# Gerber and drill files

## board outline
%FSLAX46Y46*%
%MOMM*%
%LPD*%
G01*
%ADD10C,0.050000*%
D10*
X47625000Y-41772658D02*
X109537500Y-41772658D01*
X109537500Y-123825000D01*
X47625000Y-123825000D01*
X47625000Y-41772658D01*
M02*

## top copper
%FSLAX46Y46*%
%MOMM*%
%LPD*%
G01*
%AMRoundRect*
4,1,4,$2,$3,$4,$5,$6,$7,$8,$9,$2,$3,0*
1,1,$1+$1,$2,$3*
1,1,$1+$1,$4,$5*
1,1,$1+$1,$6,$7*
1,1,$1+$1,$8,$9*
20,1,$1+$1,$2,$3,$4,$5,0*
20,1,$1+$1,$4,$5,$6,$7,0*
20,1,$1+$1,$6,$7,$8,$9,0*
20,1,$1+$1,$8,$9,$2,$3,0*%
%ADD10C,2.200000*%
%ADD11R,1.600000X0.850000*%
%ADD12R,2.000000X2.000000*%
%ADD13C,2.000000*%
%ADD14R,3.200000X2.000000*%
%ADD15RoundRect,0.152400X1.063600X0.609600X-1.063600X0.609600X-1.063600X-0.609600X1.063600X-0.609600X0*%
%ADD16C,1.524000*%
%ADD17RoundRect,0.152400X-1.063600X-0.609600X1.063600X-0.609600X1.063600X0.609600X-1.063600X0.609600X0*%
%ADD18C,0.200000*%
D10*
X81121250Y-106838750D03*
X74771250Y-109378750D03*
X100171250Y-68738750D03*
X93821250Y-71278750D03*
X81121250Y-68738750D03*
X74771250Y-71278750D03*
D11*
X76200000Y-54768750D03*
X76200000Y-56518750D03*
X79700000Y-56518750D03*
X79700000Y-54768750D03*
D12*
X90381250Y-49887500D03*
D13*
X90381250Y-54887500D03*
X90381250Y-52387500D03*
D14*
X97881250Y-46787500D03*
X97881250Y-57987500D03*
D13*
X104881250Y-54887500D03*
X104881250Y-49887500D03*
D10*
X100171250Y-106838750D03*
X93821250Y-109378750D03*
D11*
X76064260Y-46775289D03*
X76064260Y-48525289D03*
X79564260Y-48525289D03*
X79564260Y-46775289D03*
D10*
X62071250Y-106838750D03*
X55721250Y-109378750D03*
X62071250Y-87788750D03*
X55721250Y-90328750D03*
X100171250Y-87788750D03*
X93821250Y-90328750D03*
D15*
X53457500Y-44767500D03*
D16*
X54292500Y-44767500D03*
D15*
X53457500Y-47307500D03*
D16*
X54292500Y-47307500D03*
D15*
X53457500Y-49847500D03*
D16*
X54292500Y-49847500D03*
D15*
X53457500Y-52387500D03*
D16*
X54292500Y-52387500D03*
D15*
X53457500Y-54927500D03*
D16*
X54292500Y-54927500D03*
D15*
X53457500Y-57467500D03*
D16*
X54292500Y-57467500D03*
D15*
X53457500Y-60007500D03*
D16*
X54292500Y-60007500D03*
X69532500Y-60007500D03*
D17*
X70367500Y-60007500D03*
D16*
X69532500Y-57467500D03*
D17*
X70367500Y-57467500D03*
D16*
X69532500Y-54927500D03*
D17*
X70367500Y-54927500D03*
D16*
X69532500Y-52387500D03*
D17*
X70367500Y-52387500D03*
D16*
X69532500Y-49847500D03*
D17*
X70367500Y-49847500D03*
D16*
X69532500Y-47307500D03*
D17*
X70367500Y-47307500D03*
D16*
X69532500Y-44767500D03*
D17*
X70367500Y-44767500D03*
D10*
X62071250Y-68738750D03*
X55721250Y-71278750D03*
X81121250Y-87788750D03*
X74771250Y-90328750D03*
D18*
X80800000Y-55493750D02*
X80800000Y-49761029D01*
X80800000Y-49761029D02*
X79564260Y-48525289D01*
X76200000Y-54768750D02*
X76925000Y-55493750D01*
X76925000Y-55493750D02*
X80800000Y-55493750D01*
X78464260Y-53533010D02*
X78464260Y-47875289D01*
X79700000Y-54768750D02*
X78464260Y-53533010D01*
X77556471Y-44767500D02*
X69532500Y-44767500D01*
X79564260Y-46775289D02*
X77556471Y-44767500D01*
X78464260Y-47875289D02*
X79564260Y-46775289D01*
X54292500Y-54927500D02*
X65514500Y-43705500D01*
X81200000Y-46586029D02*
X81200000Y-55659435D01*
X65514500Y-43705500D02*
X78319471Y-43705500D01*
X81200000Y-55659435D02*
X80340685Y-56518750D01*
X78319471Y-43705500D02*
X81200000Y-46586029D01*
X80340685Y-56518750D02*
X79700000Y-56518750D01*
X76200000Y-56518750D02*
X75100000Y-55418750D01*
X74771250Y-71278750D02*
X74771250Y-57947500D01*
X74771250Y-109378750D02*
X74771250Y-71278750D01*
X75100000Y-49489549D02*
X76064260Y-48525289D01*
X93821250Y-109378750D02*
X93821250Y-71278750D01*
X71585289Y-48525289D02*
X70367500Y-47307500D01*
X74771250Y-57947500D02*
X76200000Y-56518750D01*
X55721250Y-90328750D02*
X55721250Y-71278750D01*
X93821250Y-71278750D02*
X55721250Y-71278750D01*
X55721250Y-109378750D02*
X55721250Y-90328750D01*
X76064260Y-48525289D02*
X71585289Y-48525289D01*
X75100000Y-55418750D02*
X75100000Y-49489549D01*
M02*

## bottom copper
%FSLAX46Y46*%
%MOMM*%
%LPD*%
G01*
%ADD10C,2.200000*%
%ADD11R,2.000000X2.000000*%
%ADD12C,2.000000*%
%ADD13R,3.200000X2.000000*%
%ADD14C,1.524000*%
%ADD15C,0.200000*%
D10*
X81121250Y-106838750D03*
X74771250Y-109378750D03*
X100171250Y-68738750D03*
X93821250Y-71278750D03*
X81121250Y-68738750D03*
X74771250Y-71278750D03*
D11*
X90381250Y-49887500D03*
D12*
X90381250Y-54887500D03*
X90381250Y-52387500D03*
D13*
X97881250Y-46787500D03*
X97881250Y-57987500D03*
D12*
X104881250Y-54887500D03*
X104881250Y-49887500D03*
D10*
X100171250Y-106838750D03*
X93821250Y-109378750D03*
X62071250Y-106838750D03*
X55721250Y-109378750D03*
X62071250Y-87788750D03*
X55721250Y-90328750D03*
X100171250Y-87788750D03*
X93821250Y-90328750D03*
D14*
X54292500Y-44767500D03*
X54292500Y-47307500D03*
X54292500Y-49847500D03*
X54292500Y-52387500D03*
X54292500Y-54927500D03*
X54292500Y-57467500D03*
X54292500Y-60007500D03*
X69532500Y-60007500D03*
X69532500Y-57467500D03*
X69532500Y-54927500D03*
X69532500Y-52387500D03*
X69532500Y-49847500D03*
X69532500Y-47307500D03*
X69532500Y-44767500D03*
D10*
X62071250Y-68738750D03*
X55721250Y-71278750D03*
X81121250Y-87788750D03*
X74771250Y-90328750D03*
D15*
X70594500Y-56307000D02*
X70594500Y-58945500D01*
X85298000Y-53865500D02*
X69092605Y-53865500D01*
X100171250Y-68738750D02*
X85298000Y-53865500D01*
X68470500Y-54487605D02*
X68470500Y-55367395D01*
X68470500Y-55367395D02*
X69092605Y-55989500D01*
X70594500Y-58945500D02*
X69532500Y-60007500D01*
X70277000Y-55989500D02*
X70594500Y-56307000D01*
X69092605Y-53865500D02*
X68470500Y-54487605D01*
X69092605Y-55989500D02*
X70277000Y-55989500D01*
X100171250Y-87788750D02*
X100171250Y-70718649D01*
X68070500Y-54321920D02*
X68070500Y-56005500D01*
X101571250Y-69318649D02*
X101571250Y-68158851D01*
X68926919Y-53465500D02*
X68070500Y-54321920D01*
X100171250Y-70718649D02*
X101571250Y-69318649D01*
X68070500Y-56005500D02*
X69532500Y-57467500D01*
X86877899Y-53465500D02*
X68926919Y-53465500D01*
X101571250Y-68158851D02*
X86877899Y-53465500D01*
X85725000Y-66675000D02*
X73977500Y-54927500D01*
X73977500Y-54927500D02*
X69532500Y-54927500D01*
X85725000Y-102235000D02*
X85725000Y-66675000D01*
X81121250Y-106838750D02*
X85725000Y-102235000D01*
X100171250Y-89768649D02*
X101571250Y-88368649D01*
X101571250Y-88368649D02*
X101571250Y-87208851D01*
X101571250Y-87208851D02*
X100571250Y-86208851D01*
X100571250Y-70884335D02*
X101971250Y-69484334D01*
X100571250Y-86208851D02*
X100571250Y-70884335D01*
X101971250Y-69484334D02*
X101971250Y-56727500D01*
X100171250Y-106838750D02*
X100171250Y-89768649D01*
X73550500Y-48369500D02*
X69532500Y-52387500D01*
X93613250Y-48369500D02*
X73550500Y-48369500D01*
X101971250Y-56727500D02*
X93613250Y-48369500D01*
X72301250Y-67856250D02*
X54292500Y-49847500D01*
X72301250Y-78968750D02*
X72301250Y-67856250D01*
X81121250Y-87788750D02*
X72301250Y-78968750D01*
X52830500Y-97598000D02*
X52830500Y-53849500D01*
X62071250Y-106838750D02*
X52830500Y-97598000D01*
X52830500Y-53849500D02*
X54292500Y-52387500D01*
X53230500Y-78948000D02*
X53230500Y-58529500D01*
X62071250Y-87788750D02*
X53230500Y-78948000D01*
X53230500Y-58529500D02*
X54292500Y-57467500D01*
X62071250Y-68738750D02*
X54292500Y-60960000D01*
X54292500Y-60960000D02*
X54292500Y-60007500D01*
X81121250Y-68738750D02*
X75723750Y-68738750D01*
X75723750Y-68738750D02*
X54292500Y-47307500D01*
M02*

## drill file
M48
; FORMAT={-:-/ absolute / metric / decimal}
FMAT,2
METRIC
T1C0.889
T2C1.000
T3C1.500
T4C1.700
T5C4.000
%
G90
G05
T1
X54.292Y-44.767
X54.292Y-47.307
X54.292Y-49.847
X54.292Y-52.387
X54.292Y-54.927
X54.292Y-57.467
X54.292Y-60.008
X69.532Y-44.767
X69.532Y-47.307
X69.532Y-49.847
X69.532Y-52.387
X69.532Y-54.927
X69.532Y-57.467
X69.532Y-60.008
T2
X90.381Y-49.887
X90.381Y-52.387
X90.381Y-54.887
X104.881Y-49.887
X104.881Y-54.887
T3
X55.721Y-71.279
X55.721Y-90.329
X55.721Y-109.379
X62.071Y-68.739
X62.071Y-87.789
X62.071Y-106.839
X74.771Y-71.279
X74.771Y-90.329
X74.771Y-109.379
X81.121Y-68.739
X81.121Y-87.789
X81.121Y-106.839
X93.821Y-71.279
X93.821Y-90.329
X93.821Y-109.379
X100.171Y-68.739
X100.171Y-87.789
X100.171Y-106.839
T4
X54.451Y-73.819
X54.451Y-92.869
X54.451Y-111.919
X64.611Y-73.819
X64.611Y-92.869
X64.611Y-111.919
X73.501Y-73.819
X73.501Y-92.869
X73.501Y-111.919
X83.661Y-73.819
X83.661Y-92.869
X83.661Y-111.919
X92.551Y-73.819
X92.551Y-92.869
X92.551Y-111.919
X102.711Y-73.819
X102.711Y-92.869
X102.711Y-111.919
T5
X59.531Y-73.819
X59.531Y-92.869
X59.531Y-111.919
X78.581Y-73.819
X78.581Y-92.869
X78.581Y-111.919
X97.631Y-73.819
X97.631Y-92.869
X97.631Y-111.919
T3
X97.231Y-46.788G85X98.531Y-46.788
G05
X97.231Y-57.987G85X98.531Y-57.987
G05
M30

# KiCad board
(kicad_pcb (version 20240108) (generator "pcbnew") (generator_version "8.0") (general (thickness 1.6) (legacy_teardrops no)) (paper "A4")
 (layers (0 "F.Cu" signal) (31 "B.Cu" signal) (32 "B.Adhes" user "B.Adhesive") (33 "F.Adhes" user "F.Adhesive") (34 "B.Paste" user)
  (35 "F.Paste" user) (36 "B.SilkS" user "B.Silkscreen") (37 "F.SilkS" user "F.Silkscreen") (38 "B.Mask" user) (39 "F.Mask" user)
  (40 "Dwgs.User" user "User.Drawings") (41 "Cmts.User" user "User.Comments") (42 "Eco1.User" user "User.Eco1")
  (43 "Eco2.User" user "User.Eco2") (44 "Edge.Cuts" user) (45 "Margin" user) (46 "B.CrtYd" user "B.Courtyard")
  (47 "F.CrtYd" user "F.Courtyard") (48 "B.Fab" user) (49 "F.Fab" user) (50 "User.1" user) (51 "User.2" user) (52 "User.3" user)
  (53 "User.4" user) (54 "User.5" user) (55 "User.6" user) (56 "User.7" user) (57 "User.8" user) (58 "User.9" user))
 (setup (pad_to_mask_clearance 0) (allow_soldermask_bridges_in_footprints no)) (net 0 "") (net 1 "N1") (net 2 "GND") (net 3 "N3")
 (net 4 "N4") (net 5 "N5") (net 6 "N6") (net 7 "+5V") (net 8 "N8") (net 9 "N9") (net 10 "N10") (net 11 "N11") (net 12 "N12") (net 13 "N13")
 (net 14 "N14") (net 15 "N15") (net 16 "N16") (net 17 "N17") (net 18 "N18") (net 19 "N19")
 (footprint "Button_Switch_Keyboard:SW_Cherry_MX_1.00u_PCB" (layer "F.Cu") (at 81.12125 106.83875)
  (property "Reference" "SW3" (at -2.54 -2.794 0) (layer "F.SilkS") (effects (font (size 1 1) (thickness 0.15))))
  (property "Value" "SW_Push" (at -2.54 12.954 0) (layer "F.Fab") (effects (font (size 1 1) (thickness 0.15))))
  (pad "" np_thru_hole circle (at -7.62 5.08) (size 1.7 1.7) (drill 1.7) (layers "*.Cu" "*.Mask"))
  (pad "" np_thru_hole circle (at -2.54 5.08) (size 4 4) (drill 4) (layers "*.Cu" "*.Mask"))
  (pad "" np_thru_hole circle (at 2.54 5.08) (size 1.7 1.7) (drill 1.7) (layers "*.Cu" "*.Mask"))
  (pad "1" thru_hole circle (at 0 0) (size 2.2 2.2) (drill 1.5) (layers "*.Cu" "*.Mask") (remove_unused_layers no) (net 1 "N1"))
  (pad "2" thru_hole circle (at -6.35 2.54) (size 2.2 2.2) (drill 1.5) (layers "*.Cu" "*.Mask") (remove_unused_layers no) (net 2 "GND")))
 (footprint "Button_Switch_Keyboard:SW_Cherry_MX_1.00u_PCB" (layer "F.Cu") (at 100.17125 68.73875)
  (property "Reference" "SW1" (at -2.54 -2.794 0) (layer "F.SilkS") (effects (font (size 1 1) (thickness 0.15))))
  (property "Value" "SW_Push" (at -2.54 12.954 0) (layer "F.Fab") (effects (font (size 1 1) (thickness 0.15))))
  (pad "" np_thru_hole circle (at -7.62 5.08) (size 1.7 1.7) (drill 1.7) (layers "*.Cu" "*.Mask"))
  (pad "" np_thru_hole circle (at -2.54 5.08) (size 4 4) (drill 4) (layers "*.Cu" "*.Mask"))
  (pad "" np_thru_hole circle (at 2.54 5.08) (size 1.7 1.7) (drill 1.7) (layers "*.Cu" "*.Mask"))
  (pad "1" thru_hole circle (at 0 0) (size 2.2 2.2) (drill 1.5) (layers "*.Cu" "*.Mask") (remove_unused_layers no) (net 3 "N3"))
  (pad "2" thru_hole circle (at -6.35 2.54) (size 2.2 2.2) (drill 1.5) (layers "*.Cu" "*.Mask") (remove_unused_layers no) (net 2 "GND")))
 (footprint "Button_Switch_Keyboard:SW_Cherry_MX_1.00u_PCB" (layer "F.Cu") (at 81.12125 68.73875)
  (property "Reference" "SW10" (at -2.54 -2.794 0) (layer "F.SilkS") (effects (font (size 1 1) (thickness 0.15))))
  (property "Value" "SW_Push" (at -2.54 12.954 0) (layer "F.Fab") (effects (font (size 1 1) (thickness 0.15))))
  (pad "" np_thru_hole circle (at -7.62 5.08) (size 1.7 1.7) (drill 1.7) (layers "*.Cu" "*.Mask"))
  (pad "" np_thru_hole circle (at -2.54 5.08) (size 4 4) (drill 4) (layers "*.Cu" "*.Mask"))
  (pad "" np_thru_hole circle (at 2.54 5.08) (size 1.7 1.7) (drill 1.7) (layers "*.Cu" "*.Mask"))
  (pad "1" thru_hole circle (at 0 0) (size 2.2 2.2) (drill 1.5) (layers "*.Cu" "*.Mask") (remove_unused_layers no) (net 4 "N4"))
  (pad "2" thru_hole circle (at -6.35 2.54) (size 2.2 2.2) (drill 1.5) (layers "*.Cu" "*.Mask") (remove_unused_layers no) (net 2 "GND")))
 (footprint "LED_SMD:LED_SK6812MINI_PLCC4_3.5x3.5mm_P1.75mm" (layer "F.Cu") (at 77.95 55.64375)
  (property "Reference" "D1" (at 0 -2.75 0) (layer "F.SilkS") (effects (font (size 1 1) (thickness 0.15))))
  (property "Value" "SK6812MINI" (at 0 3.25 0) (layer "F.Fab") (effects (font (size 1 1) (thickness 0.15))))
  (pad "1" smd rect (at -1.75 -0.875) (size 1.6 0.85) (layers "F.Cu" "F.Paste" "F.Mask") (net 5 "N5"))
  (pad "2" smd rect (at -1.75 0.875) (size 1.6 0.85) (layers "F.Cu" "F.Paste" "F.Mask") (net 2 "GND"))
  (pad "3" smd rect (at 1.75 0.875) (size 1.6 0.85) (layers "F.Cu" "F.Paste" "F.Mask") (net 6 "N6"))
  (pad "4" smd rect (at 1.75 -0.875) (size 1.6 0.85) (layers "F.Cu" "F.Paste" "F.Mask") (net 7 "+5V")))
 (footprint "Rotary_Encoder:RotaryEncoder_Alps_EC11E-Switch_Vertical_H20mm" (layer "F.Cu") (at 90.38125 49.8875)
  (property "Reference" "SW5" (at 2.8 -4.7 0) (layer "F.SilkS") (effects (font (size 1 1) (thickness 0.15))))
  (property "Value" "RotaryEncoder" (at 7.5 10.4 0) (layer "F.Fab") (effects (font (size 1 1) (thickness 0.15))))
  (pad "A" thru_hole rect (at 0 0) (size 2 2) (drill 1) (layers "*.Cu" "*.Mask") (remove_unused_layers no) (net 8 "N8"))
  (pad "B" thru_hole circle (at 0 5) (size 2 2) (drill 1) (layers "*.Cu" "*.Mask") (remove_unused_layers no) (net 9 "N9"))
  (pad "C" thru_hole circle (at 0 2.5) (size 2 2) (drill 1) (layers "*.Cu" "*.Mask") (remove_unused_layers no) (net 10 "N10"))
  (pad "MP" thru_hole rect (at 7.5 -3.1) (size 3.2 2) (drill oval 2.8 1.5) (layers "*.Cu" "*.Mask") (remove_unused_layers no))
  (pad "MP" thru_hole rect (at 7.5 8.1) (size 3.2 2) (drill oval 2.8 1.5) (layers "*.Cu" "*.Mask") (remove_unused_layers no))
  (pad "S1" thru_hole circle (at 14.5 5) (size 2 2) (drill 1) (layers "*.Cu" "*.Mask") (remove_unused_layers no))
  (pad "S2" thru_hole circle (at 14.5 0) (size 2 2) (drill 1) (layers "*.Cu" "*.Mask") (remove_unused_layers no)))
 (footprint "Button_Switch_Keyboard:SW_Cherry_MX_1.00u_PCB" (layer "F.Cu") (at 100.17125 106.83875)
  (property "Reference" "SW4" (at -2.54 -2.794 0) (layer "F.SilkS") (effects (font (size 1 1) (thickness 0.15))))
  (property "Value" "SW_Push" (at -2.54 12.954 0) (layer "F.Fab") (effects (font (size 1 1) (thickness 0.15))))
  (pad "" np_thru_hole circle (at -7.62 5.08) (size 1.7 1.7) (drill 1.7) (layers "*.Cu" "*.Mask"))
  (pad "" np_thru_hole circle (at -2.54 5.08) (size 4 4) (drill 4) (layers "*.Cu" "*.Mask"))
  (pad "" np_thru_hole circle (at 2.54 5.08) (size 1.7 1.7) (drill 1.7) (layers "*.Cu" "*.Mask"))
  (pad "1" thru_hole circle (at 0 0) (size 2.2 2.2) (drill 1.5) (layers "*.Cu" "*.Mask") (remove_unused_layers no) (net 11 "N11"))
  (pad "2" thru_hole circle (at -6.35 2.54) (size 2.2 2.2) (drill 1.5) (layers "*.Cu" "*.Mask") (remove_unused_layers no) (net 2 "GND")))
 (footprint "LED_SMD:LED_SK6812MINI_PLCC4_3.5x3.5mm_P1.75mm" (layer "F.Cu") (at 77.81426 47.650289)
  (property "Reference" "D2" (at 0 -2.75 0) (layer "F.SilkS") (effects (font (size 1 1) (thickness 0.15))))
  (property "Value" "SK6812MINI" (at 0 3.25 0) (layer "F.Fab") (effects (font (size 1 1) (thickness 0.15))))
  (pad "1" smd rect (at -1.75 -0.875) (size 1.6 0.85) (layers "F.Cu" "F.Paste" "F.Mask") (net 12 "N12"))
  (pad "2" smd rect (at -1.75 0.875) (size 1.6 0.85) (layers "F.Cu" "F.Paste" "F.Mask") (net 2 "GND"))
  (pad "3" smd rect (at 1.75 0.875) (size 1.6 0.85) (layers "F.Cu" "F.Paste" "F.Mask") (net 5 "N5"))
  (pad "4" smd rect (at 1.75 -0.875) (size 1.6 0.85) (layers "F.Cu" "F.Paste" "F.Mask") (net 7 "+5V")))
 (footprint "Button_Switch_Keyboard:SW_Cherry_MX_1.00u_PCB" (layer "F.Cu") (at 62.07125 106.83875)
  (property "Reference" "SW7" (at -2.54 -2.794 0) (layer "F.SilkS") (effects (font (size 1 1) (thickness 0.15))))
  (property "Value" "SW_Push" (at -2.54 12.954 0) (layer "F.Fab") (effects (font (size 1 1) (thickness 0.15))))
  (pad "" np_thru_hole circle (at -7.62 5.08) (size 1.7 1.7) (drill 1.7) (layers "*.Cu" "*.Mask"))
  (pad "" np_thru_hole circle (at -2.54 5.08) (size 4 4) (drill 4) (layers "*.Cu" "*.Mask"))
  (pad "" np_thru_hole circle (at 2.54 5.08) (size 1.7 1.7) (drill 1.7) (layers "*.Cu" "*.Mask"))
  (pad "1" thru_hole circle (at 0 0) (size 2.2 2.2) (drill 1.5) (layers "*.Cu" "*.Mask") (remove_unused_layers no) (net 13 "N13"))
  (pad "2" thru_hole circle (at -6.35 2.54) (size 2.2 2.2) (drill 1.5) (layers "*.Cu" "*.Mask") (remove_unused_layers no) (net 2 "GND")))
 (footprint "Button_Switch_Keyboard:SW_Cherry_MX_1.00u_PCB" (layer "F.Cu") (at 62.07125 87.78875)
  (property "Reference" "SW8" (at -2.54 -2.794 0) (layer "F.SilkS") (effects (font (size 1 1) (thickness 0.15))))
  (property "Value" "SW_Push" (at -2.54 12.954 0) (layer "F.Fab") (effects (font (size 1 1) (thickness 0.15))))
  (pad "" np_thru_hole circle (at -7.62 5.08) (size 1.7 1.7) (drill 1.7) (layers "*.Cu" "*.Mask"))
  (pad "" np_thru_hole circle (at -2.54 5.08) (size 4 4) (drill 4) (layers "*.Cu" "*.Mask"))
  (pad "" np_thru_hole circle (at 2.54 5.08) (size 1.7 1.7) (drill 1.7) (layers "*.Cu" "*.Mask"))
  (pad "1" thru_hole circle (at 0 0) (size 2.2 2.2) (drill 1.5) (layers "*.Cu" "*.Mask") (remove_unused_layers no) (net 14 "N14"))
  (pad "2" thru_hole circle (at -6.35 2.54) (size 2.2 2.2) (drill 1.5) (layers "*.Cu" "*.Mask") (remove_unused_layers no) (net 2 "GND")))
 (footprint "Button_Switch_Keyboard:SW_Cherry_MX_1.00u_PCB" (layer "F.Cu") (at 100.17125 87.78875)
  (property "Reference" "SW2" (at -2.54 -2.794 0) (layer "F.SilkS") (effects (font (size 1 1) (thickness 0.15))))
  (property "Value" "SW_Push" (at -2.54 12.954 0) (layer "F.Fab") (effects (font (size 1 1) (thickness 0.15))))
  (pad "" np_thru_hole circle (at -7.62 5.08) (size 1.7 1.7) (drill 1.7) (layers "*.Cu" "*.Mask"))
  (pad "" np_thru_hole circle (at -2.54 5.08) (size 4 4) (drill 4) (layers "*.Cu" "*.Mask"))
  (pad "" np_thru_hole circle (at 2.54 5.08) (size 1.7 1.7) (drill 1.7) (layers "*.Cu" "*.Mask"))
  (pad "1" thru_hole circle (at 0 0) (size 2.2 2.2) (drill 1.5) (layers "*.Cu" "*.Mask") (remove_unused_layers no) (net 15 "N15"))
  (pad "2" thru_hole circle (at -6.35 2.54) (size 2.2 2.2) (drill 1.5) (layers "*.Cu" "*.Mask") (remove_unused_layers no) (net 2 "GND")))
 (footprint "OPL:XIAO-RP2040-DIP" (layer "F.Cu") (at 61.9125 52.3875)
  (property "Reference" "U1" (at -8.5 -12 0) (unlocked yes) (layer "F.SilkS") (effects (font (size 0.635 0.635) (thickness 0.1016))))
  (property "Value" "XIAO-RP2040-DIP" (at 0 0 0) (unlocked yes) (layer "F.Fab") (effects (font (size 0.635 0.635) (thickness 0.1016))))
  (pad "1" smd roundrect (at -8.455 -7.62 180) (size 2.432 1.524) (layers "F.Cu" "F.Mask") (roundrect_rratio 0.1) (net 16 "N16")
   (thermal_bridge_angle 45))
  (pad "1" thru_hole circle (at -7.62 -7.62 180) (size 1.524 1.524) (drill 0.889) (layers "*.Cu" "*.Mask") (remove_unused_layers no)
   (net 16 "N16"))
  (pad "2" smd roundrect (at -8.455 -5.08 180) (size 2.432 1.524) (layers "F.Cu" "F.Mask") (roundrect_rratio 0.1) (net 4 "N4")
   (thermal_bridge_angle 45))
  (pad "2" thru_hole circle (at -7.62 -5.08 180) (size 1.524 1.524) (drill 0.889) (layers "*.Cu" "*.Mask") (remove_unused_layers no)
   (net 4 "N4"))
  (pad "3" smd roundrect (at -8.455 -2.54 180) (size 2.432 1.524) (layers "F.Cu" "F.Mask") (roundrect_rratio 0.1) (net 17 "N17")
   (thermal_bridge_angle 45))
  (pad "3" thru_hole circle (at -7.62 -2.54 180) (size 1.524 1.524) (drill 0.889) (layers "*.Cu" "*.Mask") (remove_unused_layers no)
   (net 17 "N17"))
  (pad "4" smd roundrect (at -8.455 0 180) (size 2.432 1.524) (layers "F.Cu" "F.Mask") (roundrect_rratio 0.1) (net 13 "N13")
   (thermal_bridge_angle 45))
  (pad "4" thru_hole circle (at -7.62 0 180) (size 1.524 1.524) (drill 0.889) (layers "*.Cu" "*.Mask") (remove_unused_layers no)
   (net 13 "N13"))
  (pad "5" smd roundrect (at -8.455 2.54 180) (size 2.432 1.524) (layers "F.Cu" "F.Mask") (roundrect_rratio 0.1) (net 6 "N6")
   (thermal_bridge_angle 45))
  (pad "5" thru_hole circle (at -7.62 2.54 180) (size 1.524 1.524) (drill 0.889) (layers "*.Cu" "*.Mask") (remove_unused_layers no)
   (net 6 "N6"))
  (pad "6" smd roundrect (at -8.455 5.08 180) (size 2.432 1.524) (layers "F.Cu" "F.Mask") (roundrect_rratio 0.1) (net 14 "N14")
   (thermal_bridge_angle 45))
  (pad "6" thru_hole circle (at -7.62 5.08 180) (size 1.524 1.524) (drill 0.889) (layers "*.Cu" "*.Mask") (remove_unused_layers no)
   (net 14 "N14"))
  (pad "7" smd roundrect (at -8.455 7.62 180) (size 2.432 1.524) (layers "F.Cu" "F.Mask") (roundrect_rratio 0.1) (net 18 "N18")
   (thermal_bridge_angle 45))
  (pad "7" thru_hole circle (at -7.62 7.62 180) (size 1.524 1.524) (drill 0.889) (layers "*.Cu" "*.Mask") (remove_unused_layers no)
   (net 18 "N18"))
  (pad "8" thru_hole circle (at 7.62 7.62) (size 1.524 1.524) (drill 0.889) (layers "*.Cu" "*.Mask") (remove_unused_layers no) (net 3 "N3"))
  (pad "8" smd roundrect (at 8.455 7.62) (size 2.432 1.524) (layers "F.Cu" "F.Mask") (roundrect_rratio 0.1) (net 3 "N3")
   (thermal_bridge_angle 45))
  (pad "9" thru_hole circle (at 7.62 5.08) (size 1.524 1.524) (drill 0.889) (layers "*.Cu" "*.Mask") (remove_unused_layers no)
   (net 15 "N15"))
  (pad "9" smd roundrect (at 8.455 5.08) (size 2.432 1.524) (layers "F.Cu" "F.Mask") (roundrect_rratio 0.1) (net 15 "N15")
   (thermal_bridge_angle 45))
  (pad "10" thru_hole circle (at 7.62 2.54) (size 1.524 1.524) (drill 0.889) (layers "*.Cu" "*.Mask") (remove_unused_layers no) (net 1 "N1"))
  (pad "10" smd roundrect (at 8.455 2.54) (size 2.432 1.524) (layers "F.Cu" "F.Mask") (roundrect_rratio 0.1) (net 1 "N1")
   (thermal_bridge_angle 45))
  (pad "11" thru_hole circle (at 7.62 0) (size 1.524 1.524) (drill 0.889) (layers "*.Cu" "*.Mask") (remove_unused_layers no) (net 11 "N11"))
  (pad "11" smd roundrect (at 8.455 0) (size 2.432 1.524) (layers "F.Cu" "F.Mask") (roundrect_rratio 0.1) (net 11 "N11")
   (thermal_bridge_angle 45))
  (pad "12" thru_hole circle (at 7.62 -2.54) (size 1.524 1.524) (drill 0.889) (layers "*.Cu" "*.Mask") (remove_unused_layers no)
   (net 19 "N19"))
  (pad "12" smd roundrect (at 8.455 -2.54) (size 2.432 1.524) (layers "F.Cu" "F.Mask") (roundrect_rratio 0.1) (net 19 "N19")
   (thermal_bridge_angle 45))
  (pad "13" thru_hole circle (at 7.62 -5.08) (size 1.524 1.524) (drill 0.889) (layers "*.Cu" "*.Mask") (remove_unused_layers no)
   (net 2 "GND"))
  (pad "13" smd roundrect (at 8.455 -5.08) (size 2.432 1.524) (layers "F.Cu" "F.Mask") (roundrect_rratio 0.1) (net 2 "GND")
   (thermal_bridge_angle 45))
  (pad "14" thru_hole circle (at 7.62 -7.62) (size 1.524 1.524) (drill 0.889) (layers "*.Cu" "*.Mask") (remove_unused_layers no)
   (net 7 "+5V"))
  (pad "14" smd roundrect (at 8.455 -7.62) (size 2.432 1.524) (layers "F.Cu" "F.Mask") (roundrect_rratio 0.1) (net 7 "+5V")
   (thermal_bridge_angle 45)))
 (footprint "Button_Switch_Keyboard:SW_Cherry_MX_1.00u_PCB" (layer "F.Cu") (at 62.07125 68.73875)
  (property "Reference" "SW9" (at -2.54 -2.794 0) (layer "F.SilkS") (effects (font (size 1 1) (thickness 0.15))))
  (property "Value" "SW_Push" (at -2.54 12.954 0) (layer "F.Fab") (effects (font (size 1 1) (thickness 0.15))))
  (pad "" np_thru_hole circle (at -7.62 5.08) (size 1.7 1.7) (drill 1.7) (layers "*.Cu" "*.Mask"))
  (pad "" np_thru_hole circle (at -2.54 5.08) (size 4 4) (drill 4) (layers "*.Cu" "*.Mask"))
  (pad "" np_thru_hole circle (at 2.54 5.08) (size 1.7 1.7) (drill 1.7) (layers "*.Cu" "*.Mask"))
  (pad "1" thru_hole circle (at 0 0) (size 2.2 2.2) (drill 1.5) (layers "*.Cu" "*.Mask") (remove_unused_layers no) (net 18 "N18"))
  (pad "2" thru_hole circle (at -6.35 2.54) (size 2.2 2.2) (drill 1.5) (layers "*.Cu" "*.Mask") (remove_unused_layers no) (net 2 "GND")))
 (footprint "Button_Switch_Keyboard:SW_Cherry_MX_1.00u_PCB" (layer "F.Cu") (at 81.12125 87.78875)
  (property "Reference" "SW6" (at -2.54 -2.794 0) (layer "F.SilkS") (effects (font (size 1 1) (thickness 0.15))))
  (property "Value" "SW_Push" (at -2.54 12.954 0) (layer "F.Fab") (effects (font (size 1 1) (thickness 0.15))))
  (pad "" np_thru_hole circle (at -7.62 5.08) (size 1.7 1.7) (drill 1.7) (layers "*.Cu" "*.Mask"))
  (pad "" np_thru_hole circle (at -2.54 5.08) (size 4 4) (drill 4) (layers "*.Cu" "*.Mask"))
  (pad "" np_thru_hole circle (at 2.54 5.08) (size 1.7 1.7) (drill 1.7) (layers "*.Cu" "*.Mask"))
  (pad "1" thru_hole circle (at 0 0) (size 2.2 2.2) (drill 1.5) (layers "*.Cu" "*.Mask") (remove_unused_layers no) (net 17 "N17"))
  (pad "2" thru_hole circle (at -6.35 2.54) (size 2.2 2.2) (drill 1.5) (layers "*.Cu" "*.Mask") (remove_unused_layers no) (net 2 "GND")))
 (gr_rect (start 47.625 41.772658) (end 109.5375 123.825) (stroke (width 0.05) (type default)) (fill none) (layer "Edge.Cuts"))
 (segment (start 80.8 55.49375) (end 80.8 49.761029) (width 0.2) (layer "F.Cu") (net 5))
 (segment (start 80.8 49.761029) (end 79.56426 48.525289) (width 0.2) (layer "F.Cu") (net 5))
 (segment (start 76.2 54.76875) (end 76.925 55.49375) (width 0.2) (layer "F.Cu") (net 5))
 (segment (start 76.925 55.49375) (end 80.8 55.49375) (width 0.2) (layer "F.Cu") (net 5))
 (segment (start 78.46426 53.53301) (end 78.46426 47.875289) (width 0.2) (layer "F.Cu") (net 7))
 (segment (start 79.7 54.76875) (end 78.46426 53.53301) (width 0.2) (layer "F.Cu") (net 7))
 (segment (start 77.556471 44.7675) (end 69.5325 44.7675) (width 0.2) (layer "F.Cu") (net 7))
 (segment (start 79.56426 46.775289) (end 77.556471 44.7675) (width 0.2) (layer "F.Cu") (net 7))
 (segment (start 78.46426 47.875289) (end 79.56426 46.775289) (width 0.2) (layer "F.Cu") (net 7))
 (segment (start 54.2925 54.9275) (end 65.5145 43.7055) (width 0.2) (layer "F.Cu") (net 6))
 (segment (start 81.2 46.586029) (end 81.2 55.659435) (width 0.2) (layer "F.Cu") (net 6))
 (segment (start 65.5145 43.7055) (end 78.319471 43.7055) (width 0.2) (layer "F.Cu") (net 6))
 (segment (start 81.2 55.659435) (end 80.340685 56.51875) (width 0.2) (layer "F.Cu") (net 6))
 (segment (start 78.319471 43.7055) (end 81.2 46.586029) (width 0.2) (layer "F.Cu") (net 6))
 (segment (start 80.340685 56.51875) (end 79.7 56.51875) (width 0.2) (layer "F.Cu") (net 6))
 (segment (start 76.2 56.51875) (end 75.1 55.41875) (width 0.2) (layer "F.Cu") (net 2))
 (segment (start 74.77125 71.27875) (end 74.77125 57.9475) (width 0.2) (layer "F.Cu") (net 2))
 (segment (start 74.77125 109.37875) (end 74.77125 71.27875) (width 0.2) (layer "F.Cu") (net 2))
 (segment (start 75.1 49.489549) (end 76.06426 48.525289) (width 0.2) (layer "F.Cu") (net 2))
 (segment (start 93.82125 109.37875) (end 93.82125 71.27875) (width 0.2) (layer "F.Cu") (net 2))
 (segment (start 71.585289 48.525289) (end 70.3675 47.3075) (width 0.2) (layer "F.Cu") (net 2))
 (segment (start 74.77125 57.9475) (end 76.2 56.51875) (width 0.2) (layer "F.Cu") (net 2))
 (segment (start 55.72125 90.32875) (end 55.72125 71.27875) (width 0.2) (layer "F.Cu") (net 2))
 (segment (start 93.82125 71.27875) (end 55.72125 71.27875) (width 0.2) (layer "F.Cu") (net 2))
 (segment (start 55.72125 109.37875) (end 55.72125 90.32875) (width 0.2) (layer "F.Cu") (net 2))
 (segment (start 76.06426 48.525289) (end 71.585289 48.525289) (width 0.2) (layer "F.Cu") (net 2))
 (segment (start 75.1 55.41875) (end 75.1 49.489549) (width 0.2) (layer "F.Cu") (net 2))
 (segment (start 70.5945 56.307) (end 70.5945 58.9455) (width 0.2) (layer "B.Cu") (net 3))
 (segment (start 85.298 53.8655) (end 69.092605 53.8655) (width 0.2) (layer "B.Cu") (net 3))
 (segment (start 100.17125 68.73875) (end 85.298 53.8655) (width 0.2) (layer "B.Cu") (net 3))
 (segment (start 68.4705 54.487605) (end 68.4705 55.367395) (width 0.2) (layer "B.Cu") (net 3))
 (segment (start 68.4705 55.367395) (end 69.092605 55.9895) (width 0.2) (layer "B.Cu") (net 3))
 (segment (start 70.5945 58.9455) (end 69.5325 60.0075) (width 0.2) (layer "B.Cu") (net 3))
 (segment (start 70.277 55.9895) (end 70.5945 56.307) (width 0.2) (layer "B.Cu") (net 3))
 (segment (start 69.092605 53.8655) (end 68.4705 54.487605) (width 0.2) (layer "B.Cu") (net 3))
 (segment (start 69.092605 55.9895) (end 70.277 55.9895) (width 0.2) (layer "B.Cu") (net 3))
 (segment (start 100.17125 87.78875) (end 100.17125 70.718649) (width 0.2) (layer "B.Cu") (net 15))
 (segment (start 68.0705 54.32192) (end 68.0705 56.0055) (width 0.2) (layer "B.Cu") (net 15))
 (segment (start 101.57125 69.318649) (end 101.57125 68.158851) (width 0.2) (layer "B.Cu") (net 15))
 (segment (start 68.926919 53.4655) (end 68.0705 54.32192) (width 0.2) (layer "B.Cu") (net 15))
 (segment (start 100.17125 70.718649) (end 101.57125 69.318649) (width 0.2) (layer "B.Cu") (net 15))
 (segment (start 68.0705 56.0055) (end 69.5325 57.4675) (width 0.2) (layer "B.Cu") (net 15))
 (segment (start 86.877899 53.4655) (end 68.926919 53.4655) (width 0.2) (layer "B.Cu") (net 15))
 (segment (start 101.57125 68.158851) (end 86.877899 53.4655) (width 0.2) (layer "B.Cu") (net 15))
 (segment (start 85.725 66.675) (end 73.9775 54.9275) (width 0.2) (layer "B.Cu") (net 1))
 (segment (start 73.9775 54.9275) (end 69.5325 54.9275) (width 0.2) (layer "B.Cu") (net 1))
 (segment (start 85.725 102.235) (end 85.725 66.675) (width 0.2) (layer "B.Cu") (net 1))
 (segment (start 81.12125 106.83875) (end 85.725 102.235) (width 0.2) (layer "B.Cu") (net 1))
 (segment (start 100.17125 89.768649) (end 101.57125 88.368649) (width 0.2) (layer "B.Cu") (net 11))
 (segment (start 101.57125 88.368649) (end 101.57125 87.208851) (width 0.2) (layer "B.Cu") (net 11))
 (segment (start 101.57125 87.208851) (end 100.57125 86.208851) (width 0.2) (layer "B.Cu") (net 11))
 (segment (start 100.57125 70.884335) (end 101.97125 69.484334) (width 0.2) (layer "B.Cu") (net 11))
 (segment (start 100.57125 86.208851) (end 100.57125 70.884335) (width 0.2) (layer "B.Cu") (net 11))
 (segment (start 101.97125 69.484334) (end 101.97125 56.7275) (width 0.2) (layer "B.Cu") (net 11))
 (segment (start 100.17125 106.83875) (end 100.17125 89.768649) (width 0.2) (layer "B.Cu") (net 11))
 (segment (start 73.5505 48.3695) (end 69.5325 52.3875) (width 0.2) (layer "B.Cu") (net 11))
 (segment (start 93.61325 48.3695) (end 73.5505 48.3695) (width 0.2) (layer "B.Cu") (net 11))
 (segment (start 101.97125 56.7275) (end 93.61325 48.3695) (width 0.2) (layer "B.Cu") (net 11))
 (segment (start 72.30125 67.85625) (end 54.2925 49.8475) (width 0.2) (layer "B.Cu") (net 17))
 (segment (start 72.30125 78.96875) (end 72.30125 67.85625) (width 0.2) (layer "B.Cu") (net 17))
 (segment (start 81.12125 87.78875) (end 72.30125 78.96875) (width 0.2) (layer "B.Cu") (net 17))
 (segment (start 52.8305 97.598) (end 52.8305 53.8495) (width 0.2) (layer "B.Cu") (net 13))
 (segment (start 62.07125 106.83875) (end 52.8305 97.598) (width 0.2) (layer "B.Cu") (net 13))
 (segment (start 52.8305 53.8495) (end 54.2925 52.3875) (width 0.2) (layer "B.Cu") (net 13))
 (segment (start 53.2305 78.948) (end 53.2305 58.5295) (width 0.2) (layer "B.Cu") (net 14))
 (segment (start 62.07125 87.78875) (end 53.2305 78.948) (width 0.2) (layer "B.Cu") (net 14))
 (segment (start 53.2305 58.5295) (end 54.2925 57.4675) (width 0.2) (layer "B.Cu") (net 14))
 (segment (start 62.07125 68.73875) (end 54.2925 60.96) (width 0.2) (layer "B.Cu") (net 18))
 (segment (start 54.2925 60.96) (end 54.2925 60.0075) (width 0.2) (layer "B.Cu") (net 18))
 (segment (start 81.12125 68.73875) (end 75.72375 68.73875) (width 0.2) (layer "B.Cu") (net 4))
 (segment (start 75.72375 68.73875) (end 54.2925 47.3075) (width 0.2) (layer "B.Cu") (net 4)))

